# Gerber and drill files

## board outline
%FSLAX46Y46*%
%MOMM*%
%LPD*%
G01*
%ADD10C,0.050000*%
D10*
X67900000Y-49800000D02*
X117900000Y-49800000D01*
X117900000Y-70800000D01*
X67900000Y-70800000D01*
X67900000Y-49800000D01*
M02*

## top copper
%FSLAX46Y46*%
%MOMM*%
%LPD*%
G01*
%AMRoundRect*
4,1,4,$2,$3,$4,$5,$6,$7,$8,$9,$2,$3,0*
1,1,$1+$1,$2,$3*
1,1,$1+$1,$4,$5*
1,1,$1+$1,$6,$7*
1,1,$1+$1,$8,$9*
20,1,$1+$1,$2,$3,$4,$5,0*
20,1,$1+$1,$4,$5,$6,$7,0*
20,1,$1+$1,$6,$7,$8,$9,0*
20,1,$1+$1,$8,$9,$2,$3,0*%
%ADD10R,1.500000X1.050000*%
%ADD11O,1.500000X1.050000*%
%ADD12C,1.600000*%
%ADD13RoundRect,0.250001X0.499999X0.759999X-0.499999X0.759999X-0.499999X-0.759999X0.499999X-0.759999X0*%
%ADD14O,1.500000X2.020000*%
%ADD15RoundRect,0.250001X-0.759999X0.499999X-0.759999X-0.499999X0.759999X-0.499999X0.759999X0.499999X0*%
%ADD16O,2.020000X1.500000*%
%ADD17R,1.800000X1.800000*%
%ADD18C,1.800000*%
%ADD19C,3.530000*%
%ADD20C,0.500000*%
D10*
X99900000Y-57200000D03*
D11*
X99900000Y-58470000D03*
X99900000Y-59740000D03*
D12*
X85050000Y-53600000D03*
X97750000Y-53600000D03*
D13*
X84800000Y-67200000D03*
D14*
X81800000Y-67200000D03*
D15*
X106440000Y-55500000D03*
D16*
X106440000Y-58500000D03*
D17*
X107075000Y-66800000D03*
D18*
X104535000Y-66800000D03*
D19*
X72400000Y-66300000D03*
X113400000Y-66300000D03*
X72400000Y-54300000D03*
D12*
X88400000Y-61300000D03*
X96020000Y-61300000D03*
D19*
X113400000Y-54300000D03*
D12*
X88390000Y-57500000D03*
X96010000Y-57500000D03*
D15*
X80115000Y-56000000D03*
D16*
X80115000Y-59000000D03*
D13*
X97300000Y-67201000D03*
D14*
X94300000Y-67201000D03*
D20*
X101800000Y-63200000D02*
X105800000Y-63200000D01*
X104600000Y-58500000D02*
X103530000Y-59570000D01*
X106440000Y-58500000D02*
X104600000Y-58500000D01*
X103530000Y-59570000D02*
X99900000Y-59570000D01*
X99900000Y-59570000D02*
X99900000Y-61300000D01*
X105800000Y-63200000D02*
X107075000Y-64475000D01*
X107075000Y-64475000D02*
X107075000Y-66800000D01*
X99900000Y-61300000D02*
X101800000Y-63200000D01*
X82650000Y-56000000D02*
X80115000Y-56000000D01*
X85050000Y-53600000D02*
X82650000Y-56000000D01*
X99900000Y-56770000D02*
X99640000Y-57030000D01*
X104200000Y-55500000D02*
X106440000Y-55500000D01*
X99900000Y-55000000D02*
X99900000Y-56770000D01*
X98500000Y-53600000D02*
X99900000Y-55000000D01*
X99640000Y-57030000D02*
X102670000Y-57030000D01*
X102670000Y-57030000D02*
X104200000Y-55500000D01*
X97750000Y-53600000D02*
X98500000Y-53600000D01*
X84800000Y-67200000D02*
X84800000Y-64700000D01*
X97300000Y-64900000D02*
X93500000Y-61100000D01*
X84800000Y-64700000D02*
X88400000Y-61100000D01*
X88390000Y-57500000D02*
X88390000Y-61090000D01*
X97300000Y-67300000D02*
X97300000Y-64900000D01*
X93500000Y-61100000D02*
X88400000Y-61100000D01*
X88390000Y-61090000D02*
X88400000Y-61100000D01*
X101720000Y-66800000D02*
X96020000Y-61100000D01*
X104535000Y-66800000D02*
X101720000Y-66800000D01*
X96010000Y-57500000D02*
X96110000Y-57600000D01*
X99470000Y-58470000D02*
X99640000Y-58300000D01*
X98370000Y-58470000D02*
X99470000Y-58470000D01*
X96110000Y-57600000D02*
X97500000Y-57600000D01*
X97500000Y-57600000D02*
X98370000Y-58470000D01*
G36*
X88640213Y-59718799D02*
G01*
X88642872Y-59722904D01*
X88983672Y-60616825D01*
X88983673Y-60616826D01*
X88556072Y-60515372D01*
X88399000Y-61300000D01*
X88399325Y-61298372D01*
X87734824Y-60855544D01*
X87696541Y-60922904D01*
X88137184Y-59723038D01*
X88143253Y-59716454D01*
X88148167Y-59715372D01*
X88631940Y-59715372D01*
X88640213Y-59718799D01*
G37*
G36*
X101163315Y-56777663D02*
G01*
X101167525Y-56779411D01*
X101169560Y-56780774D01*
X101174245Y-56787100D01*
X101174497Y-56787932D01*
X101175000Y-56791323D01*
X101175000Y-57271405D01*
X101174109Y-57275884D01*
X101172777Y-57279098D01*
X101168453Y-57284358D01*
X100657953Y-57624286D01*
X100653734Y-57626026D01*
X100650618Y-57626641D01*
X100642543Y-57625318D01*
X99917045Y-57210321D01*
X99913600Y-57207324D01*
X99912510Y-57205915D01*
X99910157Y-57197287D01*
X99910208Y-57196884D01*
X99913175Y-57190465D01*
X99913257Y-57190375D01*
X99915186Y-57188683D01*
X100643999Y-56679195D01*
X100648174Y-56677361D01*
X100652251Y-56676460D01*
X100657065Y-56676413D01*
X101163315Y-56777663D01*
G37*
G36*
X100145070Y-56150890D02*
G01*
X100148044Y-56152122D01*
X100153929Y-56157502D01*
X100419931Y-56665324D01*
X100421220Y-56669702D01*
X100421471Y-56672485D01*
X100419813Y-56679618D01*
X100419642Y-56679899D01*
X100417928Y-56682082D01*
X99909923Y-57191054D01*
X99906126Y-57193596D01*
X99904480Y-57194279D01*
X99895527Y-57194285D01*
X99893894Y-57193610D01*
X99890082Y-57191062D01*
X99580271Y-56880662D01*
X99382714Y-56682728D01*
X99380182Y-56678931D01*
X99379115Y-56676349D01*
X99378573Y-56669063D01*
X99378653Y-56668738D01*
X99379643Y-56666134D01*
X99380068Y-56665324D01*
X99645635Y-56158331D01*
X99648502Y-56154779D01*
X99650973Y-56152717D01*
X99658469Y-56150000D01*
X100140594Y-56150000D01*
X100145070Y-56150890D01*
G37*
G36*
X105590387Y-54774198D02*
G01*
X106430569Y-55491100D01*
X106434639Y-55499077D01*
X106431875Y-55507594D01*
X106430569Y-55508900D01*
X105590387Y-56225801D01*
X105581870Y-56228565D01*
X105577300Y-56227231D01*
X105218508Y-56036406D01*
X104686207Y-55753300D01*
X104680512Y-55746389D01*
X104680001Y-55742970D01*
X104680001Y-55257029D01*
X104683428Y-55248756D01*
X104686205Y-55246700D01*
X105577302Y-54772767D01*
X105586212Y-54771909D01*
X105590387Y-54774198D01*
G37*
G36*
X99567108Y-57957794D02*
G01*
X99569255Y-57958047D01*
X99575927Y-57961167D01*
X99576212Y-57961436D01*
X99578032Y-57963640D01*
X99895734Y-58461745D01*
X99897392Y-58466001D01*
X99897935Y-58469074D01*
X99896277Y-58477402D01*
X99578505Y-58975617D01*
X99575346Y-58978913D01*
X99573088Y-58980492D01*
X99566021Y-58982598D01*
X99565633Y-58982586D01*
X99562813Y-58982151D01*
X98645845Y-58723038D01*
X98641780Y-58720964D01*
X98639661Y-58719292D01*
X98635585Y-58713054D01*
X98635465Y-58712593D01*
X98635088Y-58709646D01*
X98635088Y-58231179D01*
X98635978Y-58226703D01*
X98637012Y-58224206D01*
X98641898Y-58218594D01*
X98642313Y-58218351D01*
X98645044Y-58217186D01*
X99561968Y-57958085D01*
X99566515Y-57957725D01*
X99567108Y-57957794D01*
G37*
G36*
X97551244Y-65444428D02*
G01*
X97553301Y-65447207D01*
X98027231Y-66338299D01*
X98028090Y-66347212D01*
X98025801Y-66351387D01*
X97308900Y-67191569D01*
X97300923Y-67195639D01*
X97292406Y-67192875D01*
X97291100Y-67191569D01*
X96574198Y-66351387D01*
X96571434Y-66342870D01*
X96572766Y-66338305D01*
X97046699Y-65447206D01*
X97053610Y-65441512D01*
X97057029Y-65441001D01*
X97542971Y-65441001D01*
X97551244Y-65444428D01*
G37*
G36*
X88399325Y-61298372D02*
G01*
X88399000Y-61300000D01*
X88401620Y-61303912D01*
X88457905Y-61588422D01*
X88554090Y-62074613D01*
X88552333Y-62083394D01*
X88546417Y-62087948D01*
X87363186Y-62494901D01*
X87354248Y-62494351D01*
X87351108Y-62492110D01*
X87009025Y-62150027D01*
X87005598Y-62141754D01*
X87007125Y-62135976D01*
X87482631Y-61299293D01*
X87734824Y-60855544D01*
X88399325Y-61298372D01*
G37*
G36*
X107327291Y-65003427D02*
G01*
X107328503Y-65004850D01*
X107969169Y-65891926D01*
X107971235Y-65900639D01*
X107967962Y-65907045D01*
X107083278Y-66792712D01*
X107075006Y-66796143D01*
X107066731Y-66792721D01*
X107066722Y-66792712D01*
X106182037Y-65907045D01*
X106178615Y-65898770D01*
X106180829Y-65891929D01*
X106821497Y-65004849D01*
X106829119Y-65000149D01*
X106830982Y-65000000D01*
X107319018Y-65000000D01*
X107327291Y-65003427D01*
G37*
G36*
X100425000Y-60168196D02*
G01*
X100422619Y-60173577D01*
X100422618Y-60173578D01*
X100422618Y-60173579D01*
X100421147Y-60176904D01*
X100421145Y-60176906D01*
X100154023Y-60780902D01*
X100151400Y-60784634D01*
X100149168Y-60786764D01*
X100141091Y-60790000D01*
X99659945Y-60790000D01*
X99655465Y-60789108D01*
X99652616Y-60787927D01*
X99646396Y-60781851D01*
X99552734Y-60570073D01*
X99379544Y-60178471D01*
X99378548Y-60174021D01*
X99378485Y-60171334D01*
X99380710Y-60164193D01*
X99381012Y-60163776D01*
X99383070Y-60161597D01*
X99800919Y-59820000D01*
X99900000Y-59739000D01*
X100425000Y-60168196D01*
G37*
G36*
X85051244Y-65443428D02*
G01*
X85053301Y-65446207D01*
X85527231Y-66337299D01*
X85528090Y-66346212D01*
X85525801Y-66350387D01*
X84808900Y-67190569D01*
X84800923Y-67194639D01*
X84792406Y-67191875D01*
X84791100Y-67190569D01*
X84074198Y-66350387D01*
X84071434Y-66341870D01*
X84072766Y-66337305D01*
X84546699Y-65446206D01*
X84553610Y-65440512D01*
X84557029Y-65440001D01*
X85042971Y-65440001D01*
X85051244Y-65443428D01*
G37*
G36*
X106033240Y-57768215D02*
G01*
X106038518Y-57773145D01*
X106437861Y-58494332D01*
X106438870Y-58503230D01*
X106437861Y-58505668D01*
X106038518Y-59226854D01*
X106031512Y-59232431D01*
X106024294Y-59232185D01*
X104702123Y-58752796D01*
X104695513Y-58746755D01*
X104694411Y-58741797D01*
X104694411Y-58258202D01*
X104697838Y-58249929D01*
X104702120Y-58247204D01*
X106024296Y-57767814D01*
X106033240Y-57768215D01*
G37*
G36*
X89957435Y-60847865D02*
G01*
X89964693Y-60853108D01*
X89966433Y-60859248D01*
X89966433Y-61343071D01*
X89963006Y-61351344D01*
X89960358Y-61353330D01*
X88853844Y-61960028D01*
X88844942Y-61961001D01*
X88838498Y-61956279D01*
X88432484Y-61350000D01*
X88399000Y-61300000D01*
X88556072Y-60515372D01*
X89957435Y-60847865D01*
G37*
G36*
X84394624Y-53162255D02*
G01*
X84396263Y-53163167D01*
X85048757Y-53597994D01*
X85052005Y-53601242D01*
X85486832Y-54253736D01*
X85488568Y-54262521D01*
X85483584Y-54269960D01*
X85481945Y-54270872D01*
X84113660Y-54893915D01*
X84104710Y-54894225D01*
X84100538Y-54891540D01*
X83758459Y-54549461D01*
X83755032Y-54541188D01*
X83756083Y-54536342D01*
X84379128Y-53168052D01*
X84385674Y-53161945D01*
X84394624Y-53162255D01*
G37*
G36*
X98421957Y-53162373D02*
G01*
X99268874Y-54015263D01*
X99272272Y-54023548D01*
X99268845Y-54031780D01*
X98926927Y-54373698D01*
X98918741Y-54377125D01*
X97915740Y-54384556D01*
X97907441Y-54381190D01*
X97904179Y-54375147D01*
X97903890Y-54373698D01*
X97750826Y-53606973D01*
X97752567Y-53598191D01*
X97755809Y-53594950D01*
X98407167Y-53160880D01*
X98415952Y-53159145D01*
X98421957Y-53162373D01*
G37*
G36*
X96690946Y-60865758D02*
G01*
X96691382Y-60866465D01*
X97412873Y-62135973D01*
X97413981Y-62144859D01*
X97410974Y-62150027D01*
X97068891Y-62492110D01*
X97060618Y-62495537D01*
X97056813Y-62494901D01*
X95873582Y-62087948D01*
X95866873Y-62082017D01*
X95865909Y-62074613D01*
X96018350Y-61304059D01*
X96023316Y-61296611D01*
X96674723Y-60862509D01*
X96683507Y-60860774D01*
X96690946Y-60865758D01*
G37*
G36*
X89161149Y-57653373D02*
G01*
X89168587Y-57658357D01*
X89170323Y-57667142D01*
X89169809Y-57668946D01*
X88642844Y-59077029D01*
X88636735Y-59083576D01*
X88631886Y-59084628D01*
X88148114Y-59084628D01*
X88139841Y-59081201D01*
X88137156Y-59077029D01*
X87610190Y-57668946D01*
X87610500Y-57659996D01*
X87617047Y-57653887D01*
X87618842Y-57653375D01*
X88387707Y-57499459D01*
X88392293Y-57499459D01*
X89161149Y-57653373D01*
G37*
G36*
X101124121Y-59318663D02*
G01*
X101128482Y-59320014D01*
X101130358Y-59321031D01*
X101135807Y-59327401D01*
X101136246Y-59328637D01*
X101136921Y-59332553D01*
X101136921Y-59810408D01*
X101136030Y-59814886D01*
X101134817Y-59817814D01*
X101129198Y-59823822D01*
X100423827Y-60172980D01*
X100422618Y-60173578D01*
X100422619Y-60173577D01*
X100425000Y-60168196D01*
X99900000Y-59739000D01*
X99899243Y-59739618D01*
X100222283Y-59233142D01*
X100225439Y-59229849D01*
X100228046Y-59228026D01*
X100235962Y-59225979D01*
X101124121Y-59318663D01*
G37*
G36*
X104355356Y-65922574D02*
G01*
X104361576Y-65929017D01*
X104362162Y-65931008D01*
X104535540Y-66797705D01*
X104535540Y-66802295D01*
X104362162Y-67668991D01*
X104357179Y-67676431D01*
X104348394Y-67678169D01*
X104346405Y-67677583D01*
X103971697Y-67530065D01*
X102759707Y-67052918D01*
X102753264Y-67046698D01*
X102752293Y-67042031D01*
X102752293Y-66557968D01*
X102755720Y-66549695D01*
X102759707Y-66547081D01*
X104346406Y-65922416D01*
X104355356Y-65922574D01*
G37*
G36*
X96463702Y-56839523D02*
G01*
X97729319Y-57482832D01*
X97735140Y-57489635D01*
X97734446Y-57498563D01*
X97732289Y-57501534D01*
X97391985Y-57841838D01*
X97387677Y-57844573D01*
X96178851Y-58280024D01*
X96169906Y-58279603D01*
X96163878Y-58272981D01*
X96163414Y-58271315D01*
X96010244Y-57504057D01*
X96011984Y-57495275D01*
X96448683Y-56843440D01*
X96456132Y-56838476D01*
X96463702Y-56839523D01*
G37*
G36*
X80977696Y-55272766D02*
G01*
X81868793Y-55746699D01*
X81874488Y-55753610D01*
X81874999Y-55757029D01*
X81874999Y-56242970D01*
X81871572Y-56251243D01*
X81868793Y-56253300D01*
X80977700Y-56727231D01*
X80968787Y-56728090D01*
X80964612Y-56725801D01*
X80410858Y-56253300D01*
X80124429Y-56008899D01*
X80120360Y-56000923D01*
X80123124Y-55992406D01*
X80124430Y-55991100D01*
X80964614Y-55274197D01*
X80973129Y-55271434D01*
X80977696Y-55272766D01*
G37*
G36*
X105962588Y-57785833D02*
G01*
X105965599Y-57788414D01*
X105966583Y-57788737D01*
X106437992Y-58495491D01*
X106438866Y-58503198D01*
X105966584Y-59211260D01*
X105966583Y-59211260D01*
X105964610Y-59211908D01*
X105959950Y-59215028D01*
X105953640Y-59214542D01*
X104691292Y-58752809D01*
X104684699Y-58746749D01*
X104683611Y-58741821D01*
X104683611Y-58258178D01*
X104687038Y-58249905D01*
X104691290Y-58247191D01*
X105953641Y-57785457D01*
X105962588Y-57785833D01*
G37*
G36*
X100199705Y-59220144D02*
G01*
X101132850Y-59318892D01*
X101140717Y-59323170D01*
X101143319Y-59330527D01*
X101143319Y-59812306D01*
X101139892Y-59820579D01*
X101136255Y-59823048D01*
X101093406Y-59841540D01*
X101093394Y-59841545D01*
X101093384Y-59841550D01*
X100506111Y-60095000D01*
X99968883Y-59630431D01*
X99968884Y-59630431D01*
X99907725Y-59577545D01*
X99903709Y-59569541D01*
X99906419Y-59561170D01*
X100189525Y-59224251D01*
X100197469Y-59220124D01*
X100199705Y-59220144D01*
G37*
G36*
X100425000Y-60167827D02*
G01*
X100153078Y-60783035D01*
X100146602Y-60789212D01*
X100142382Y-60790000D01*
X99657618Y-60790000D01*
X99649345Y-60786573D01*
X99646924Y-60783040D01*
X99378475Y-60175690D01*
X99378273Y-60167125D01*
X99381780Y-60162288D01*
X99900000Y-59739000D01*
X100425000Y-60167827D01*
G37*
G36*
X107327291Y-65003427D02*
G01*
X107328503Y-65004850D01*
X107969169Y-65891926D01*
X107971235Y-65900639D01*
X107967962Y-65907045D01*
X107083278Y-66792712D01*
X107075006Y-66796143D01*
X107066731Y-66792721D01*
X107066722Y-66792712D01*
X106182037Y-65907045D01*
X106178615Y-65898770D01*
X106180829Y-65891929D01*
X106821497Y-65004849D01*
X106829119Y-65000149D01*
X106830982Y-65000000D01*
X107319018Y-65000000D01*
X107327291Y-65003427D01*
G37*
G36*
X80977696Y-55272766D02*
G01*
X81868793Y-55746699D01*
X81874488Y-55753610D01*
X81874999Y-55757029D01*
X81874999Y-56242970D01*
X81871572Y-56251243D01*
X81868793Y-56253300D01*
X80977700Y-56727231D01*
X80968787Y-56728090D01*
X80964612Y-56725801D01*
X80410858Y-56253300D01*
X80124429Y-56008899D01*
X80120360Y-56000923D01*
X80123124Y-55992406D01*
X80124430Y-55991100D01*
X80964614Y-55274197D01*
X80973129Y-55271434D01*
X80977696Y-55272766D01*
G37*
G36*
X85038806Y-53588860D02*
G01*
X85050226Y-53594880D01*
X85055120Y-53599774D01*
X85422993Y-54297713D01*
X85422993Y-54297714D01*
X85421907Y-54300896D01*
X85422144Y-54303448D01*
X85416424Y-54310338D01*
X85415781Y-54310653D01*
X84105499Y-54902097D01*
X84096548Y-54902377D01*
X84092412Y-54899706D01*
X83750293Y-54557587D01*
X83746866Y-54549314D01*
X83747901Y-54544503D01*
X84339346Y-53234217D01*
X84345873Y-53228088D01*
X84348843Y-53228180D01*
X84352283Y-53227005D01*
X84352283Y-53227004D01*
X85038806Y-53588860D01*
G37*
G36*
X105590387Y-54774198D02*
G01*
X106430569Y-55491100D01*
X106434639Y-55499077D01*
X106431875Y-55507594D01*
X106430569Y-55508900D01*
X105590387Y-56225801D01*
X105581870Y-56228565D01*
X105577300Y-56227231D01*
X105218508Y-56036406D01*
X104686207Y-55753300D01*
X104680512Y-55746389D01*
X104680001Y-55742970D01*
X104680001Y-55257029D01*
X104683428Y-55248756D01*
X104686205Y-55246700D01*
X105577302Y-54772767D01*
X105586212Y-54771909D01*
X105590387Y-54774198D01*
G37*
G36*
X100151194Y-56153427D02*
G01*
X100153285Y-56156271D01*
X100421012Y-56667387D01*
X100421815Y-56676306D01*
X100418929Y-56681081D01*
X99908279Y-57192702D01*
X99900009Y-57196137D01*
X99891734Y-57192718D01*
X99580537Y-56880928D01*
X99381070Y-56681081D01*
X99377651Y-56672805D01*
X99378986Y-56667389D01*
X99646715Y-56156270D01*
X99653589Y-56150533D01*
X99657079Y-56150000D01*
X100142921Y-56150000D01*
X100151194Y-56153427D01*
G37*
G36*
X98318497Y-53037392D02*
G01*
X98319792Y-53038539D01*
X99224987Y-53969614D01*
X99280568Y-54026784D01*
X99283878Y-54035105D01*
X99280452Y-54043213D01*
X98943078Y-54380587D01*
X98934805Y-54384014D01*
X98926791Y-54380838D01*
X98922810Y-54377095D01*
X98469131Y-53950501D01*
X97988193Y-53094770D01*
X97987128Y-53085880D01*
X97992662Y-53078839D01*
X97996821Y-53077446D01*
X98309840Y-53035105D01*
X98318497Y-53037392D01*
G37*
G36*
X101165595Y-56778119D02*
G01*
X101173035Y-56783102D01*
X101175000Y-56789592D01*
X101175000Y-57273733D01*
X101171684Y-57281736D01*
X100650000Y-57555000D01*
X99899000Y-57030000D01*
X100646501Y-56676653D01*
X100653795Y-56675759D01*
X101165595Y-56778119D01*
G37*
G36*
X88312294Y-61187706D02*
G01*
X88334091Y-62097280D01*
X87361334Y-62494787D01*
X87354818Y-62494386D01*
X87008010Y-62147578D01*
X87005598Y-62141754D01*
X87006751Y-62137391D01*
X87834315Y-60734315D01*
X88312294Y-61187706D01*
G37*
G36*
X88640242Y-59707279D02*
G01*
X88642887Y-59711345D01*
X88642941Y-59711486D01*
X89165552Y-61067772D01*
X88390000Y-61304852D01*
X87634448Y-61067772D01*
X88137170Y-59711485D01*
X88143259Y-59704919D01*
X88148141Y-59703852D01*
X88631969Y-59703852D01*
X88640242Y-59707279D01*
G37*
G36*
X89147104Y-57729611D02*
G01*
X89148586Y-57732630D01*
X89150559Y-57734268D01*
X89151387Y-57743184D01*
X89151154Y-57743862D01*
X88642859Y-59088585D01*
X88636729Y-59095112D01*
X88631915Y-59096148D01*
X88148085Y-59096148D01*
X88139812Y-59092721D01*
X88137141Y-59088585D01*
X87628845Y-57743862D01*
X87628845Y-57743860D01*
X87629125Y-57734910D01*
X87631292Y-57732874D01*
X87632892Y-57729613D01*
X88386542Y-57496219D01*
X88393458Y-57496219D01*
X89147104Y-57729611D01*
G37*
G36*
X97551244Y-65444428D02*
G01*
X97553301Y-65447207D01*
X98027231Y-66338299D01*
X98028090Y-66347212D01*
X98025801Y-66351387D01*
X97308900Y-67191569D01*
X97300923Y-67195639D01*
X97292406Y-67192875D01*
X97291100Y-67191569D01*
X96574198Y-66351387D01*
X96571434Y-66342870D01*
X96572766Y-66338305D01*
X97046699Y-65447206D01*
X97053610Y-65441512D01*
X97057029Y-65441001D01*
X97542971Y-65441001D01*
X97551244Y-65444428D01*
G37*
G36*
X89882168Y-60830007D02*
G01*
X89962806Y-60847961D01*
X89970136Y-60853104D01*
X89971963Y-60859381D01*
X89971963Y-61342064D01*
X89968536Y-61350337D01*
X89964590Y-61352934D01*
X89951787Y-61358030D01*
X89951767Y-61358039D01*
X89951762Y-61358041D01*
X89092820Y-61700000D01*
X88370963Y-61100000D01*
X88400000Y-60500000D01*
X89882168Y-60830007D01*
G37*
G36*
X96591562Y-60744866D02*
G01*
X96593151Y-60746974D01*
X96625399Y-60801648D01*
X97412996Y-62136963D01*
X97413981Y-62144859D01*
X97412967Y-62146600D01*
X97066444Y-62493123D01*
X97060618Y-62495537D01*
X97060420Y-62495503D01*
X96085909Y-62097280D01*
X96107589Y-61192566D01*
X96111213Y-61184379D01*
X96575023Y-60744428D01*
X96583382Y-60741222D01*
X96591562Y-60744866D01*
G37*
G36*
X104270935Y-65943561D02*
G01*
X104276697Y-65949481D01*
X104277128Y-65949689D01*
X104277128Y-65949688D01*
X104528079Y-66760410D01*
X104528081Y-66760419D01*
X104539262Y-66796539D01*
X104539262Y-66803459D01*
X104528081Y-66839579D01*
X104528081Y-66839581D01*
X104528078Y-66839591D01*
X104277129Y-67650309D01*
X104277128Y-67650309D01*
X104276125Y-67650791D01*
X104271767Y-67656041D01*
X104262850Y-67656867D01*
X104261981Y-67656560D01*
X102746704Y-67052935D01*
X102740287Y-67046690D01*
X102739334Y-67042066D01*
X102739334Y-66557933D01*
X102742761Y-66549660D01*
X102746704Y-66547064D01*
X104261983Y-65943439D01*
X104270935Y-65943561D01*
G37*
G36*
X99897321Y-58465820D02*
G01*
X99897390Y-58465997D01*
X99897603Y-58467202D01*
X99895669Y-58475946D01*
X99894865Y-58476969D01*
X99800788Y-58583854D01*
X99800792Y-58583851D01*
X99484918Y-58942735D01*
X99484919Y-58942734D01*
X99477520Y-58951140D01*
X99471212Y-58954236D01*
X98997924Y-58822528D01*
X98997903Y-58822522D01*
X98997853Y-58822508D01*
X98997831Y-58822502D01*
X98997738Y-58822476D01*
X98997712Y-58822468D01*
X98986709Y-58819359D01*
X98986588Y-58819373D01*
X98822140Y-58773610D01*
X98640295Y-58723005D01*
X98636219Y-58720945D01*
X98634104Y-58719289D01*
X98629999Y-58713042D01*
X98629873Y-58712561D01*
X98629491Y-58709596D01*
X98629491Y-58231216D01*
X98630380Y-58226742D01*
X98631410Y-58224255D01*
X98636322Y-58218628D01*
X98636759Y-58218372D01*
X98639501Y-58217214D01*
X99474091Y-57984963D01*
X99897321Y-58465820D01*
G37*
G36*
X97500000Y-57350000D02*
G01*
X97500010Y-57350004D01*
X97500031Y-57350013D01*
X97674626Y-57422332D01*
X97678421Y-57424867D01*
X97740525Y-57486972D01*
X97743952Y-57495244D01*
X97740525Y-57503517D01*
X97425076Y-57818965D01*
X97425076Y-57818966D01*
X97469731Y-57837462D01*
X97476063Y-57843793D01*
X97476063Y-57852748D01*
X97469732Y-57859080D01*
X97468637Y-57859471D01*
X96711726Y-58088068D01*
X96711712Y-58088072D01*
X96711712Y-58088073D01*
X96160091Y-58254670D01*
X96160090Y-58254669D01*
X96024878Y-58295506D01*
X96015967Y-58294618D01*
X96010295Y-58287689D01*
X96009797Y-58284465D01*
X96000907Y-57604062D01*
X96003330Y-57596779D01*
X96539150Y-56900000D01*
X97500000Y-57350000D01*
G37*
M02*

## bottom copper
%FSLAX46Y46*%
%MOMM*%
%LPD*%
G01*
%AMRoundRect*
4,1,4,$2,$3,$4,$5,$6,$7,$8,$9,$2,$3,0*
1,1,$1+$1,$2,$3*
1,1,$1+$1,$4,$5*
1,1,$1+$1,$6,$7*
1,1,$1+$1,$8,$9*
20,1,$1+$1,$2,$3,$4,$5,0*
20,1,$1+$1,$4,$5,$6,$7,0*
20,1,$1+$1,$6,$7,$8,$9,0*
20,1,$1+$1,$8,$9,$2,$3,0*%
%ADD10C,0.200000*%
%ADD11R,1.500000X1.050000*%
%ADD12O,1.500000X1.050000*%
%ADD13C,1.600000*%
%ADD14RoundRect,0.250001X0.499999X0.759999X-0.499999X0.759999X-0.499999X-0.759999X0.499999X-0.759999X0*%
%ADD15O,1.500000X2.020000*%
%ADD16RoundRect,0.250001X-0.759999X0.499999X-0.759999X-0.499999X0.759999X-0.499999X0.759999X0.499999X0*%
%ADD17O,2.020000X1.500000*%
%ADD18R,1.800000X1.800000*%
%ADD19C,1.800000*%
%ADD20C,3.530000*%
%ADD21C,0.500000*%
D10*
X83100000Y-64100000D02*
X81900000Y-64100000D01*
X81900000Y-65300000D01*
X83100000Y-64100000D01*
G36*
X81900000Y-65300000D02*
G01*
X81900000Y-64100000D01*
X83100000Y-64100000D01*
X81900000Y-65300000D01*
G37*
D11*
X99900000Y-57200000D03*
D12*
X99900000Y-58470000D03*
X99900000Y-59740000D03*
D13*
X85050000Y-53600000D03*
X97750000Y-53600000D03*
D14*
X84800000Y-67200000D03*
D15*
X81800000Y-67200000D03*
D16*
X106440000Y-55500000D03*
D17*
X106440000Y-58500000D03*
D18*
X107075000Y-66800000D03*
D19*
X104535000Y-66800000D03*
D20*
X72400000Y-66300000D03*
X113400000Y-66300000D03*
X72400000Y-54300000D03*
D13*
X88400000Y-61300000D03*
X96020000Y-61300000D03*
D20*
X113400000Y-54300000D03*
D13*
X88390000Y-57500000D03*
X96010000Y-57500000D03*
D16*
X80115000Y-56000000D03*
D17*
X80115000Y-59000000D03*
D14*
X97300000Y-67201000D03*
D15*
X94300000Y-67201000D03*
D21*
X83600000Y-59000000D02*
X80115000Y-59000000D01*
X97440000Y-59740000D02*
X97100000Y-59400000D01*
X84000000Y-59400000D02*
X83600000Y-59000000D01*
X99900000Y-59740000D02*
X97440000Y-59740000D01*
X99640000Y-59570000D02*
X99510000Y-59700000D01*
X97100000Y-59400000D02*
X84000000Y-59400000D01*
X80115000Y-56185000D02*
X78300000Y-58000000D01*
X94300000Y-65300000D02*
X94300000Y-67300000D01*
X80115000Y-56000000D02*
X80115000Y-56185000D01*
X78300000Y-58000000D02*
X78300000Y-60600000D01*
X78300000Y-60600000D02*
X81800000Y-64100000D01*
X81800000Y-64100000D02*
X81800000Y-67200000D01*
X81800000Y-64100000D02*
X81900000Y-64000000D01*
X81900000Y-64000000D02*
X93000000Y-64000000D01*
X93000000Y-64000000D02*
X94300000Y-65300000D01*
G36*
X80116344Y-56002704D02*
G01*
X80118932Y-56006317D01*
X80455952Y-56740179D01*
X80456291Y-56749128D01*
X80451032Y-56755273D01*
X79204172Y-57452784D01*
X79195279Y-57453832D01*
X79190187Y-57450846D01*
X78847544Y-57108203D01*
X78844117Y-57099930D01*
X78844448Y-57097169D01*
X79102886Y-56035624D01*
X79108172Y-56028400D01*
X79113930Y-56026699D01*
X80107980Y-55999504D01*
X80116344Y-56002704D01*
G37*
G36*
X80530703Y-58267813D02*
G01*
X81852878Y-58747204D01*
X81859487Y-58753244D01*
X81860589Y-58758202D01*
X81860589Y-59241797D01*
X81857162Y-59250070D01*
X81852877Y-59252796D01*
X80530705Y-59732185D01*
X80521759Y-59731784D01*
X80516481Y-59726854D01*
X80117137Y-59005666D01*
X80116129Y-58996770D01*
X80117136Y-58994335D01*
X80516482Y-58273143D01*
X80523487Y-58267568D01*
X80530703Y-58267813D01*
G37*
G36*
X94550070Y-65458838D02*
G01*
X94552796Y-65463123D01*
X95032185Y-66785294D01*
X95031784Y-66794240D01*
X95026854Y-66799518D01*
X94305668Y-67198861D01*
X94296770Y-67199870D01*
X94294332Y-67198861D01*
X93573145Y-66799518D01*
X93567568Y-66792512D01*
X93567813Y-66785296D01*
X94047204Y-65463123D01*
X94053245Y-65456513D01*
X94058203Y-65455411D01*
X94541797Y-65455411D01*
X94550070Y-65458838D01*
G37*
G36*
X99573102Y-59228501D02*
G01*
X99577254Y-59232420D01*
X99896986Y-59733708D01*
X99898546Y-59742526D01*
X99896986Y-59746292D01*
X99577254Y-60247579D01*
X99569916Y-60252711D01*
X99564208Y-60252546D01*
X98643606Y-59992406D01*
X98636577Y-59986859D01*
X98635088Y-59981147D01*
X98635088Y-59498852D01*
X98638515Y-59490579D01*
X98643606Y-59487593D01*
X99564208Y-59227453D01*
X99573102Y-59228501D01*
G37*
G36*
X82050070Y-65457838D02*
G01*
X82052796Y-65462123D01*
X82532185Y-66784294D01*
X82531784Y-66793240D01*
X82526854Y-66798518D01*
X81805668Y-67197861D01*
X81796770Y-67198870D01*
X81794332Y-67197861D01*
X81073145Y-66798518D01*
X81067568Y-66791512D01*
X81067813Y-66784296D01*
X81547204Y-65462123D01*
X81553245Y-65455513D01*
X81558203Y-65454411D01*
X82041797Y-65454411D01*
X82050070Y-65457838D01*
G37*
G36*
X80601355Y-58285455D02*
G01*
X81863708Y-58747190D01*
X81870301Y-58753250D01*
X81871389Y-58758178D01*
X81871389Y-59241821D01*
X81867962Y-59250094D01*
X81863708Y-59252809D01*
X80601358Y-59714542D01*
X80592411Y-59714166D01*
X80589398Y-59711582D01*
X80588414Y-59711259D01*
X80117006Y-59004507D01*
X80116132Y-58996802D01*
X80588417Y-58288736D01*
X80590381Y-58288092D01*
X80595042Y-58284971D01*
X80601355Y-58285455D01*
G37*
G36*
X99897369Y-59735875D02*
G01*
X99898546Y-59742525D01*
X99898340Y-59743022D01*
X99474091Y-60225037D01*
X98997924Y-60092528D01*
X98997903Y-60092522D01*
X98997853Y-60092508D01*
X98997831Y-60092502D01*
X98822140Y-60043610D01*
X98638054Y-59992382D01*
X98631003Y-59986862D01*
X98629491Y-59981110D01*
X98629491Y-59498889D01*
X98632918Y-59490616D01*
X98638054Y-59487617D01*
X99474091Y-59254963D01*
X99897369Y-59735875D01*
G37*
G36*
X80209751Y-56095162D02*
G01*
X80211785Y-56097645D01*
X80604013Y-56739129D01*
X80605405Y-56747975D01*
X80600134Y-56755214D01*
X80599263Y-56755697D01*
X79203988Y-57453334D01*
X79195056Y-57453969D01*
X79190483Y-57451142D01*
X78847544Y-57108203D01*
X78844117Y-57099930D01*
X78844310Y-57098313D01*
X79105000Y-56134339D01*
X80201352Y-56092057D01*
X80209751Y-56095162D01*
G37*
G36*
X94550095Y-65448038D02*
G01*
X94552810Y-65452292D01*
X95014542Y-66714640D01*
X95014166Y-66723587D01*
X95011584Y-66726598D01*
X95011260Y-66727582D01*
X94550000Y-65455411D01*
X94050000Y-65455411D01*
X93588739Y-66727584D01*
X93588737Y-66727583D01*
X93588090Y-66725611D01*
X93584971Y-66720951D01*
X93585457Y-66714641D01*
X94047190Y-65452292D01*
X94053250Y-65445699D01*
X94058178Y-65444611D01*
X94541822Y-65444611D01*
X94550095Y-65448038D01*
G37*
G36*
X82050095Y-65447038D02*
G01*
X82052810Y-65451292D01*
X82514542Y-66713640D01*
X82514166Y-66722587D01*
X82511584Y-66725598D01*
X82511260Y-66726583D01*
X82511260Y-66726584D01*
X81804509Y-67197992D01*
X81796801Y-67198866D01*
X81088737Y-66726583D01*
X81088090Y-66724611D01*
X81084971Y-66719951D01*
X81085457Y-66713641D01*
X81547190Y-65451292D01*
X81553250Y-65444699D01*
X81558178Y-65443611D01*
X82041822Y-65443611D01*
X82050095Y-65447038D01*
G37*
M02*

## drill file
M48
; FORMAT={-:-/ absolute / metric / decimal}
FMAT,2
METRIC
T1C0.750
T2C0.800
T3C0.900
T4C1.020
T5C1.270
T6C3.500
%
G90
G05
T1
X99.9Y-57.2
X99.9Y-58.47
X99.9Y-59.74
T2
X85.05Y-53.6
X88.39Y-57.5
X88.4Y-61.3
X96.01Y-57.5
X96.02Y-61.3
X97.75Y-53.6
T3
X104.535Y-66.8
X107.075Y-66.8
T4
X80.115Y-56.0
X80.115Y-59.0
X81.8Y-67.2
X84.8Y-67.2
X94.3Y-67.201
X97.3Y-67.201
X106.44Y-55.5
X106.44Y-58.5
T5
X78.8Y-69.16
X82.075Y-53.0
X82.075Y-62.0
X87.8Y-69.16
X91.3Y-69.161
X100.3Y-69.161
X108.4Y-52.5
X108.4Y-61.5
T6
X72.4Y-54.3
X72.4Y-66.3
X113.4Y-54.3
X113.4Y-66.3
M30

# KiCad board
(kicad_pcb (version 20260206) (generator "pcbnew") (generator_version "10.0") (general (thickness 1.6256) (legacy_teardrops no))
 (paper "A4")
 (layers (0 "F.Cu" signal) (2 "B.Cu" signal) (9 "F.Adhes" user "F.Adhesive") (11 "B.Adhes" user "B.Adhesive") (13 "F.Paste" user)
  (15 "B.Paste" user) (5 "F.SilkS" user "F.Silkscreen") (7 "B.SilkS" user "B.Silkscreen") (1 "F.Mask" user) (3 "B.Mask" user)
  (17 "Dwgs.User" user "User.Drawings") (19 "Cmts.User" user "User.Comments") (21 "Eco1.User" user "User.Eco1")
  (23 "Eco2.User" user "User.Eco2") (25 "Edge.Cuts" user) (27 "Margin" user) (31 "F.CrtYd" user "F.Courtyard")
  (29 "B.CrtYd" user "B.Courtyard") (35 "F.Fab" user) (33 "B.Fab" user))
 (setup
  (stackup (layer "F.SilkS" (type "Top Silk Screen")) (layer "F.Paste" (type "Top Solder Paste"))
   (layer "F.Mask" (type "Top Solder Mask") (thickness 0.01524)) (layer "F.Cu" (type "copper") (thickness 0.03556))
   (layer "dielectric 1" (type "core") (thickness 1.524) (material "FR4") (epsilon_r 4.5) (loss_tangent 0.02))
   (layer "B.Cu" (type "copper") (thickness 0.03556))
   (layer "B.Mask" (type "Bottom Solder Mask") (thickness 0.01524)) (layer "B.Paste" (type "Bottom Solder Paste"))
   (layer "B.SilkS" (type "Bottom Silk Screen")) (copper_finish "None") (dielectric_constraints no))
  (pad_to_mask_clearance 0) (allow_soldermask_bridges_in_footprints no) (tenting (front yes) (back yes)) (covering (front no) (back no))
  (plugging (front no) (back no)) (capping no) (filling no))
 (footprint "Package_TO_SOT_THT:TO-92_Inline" (layer "F.Cu") (at 99.9 57.2 -90)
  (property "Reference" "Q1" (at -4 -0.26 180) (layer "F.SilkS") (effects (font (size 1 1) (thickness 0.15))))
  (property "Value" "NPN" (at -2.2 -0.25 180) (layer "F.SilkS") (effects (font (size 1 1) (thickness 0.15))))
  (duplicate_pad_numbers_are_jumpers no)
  (pad "1" thru_hole rect (at 0 0 270) (size 1.05 1.5) (drill 0.75) (layers "*.Cu" "*.Mask") (remove_unused_layers no)
   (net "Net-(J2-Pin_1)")
   (teardrops (best_length_ratio 0.5) (max_length 1) (best_width_ratio 1) (max_width 2) (curved_edges no) (filter_ratio 0.9) (enabled yes)
    (allow_two_segments yes) (prefer_zone_connections yes)))
  (pad "2" thru_hole oval (at 1.27 0 270) (size 1.05 1.5) (drill 0.75) (layers "*.Cu" "*.Mask") (remove_unused_layers no) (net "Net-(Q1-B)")
   (teardrops (best_length_ratio 0.5) (max_length 1) (best_width_ratio 1) (max_width 2) (curved_edges no) (filter_ratio 0.9) (enabled yes)
    (allow_two_segments yes) (prefer_zone_connections yes)))
  (pad "3" thru_hole oval (at 2.54 0 270) (size 1.05 1.5) (drill 0.75) (layers "*.Cu" "*.Mask") (remove_unused_layers no) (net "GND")
   (teardrops (best_length_ratio 0.5) (max_length 1) (best_width_ratio 1) (max_width 2) (curved_edges no) (filter_ratio 0.9) (enabled yes)
    (allow_two_segments yes) (prefer_zone_connections yes))))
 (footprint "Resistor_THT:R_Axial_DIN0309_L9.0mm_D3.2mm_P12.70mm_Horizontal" (layer "F.Cu") (at 85.05 53.6)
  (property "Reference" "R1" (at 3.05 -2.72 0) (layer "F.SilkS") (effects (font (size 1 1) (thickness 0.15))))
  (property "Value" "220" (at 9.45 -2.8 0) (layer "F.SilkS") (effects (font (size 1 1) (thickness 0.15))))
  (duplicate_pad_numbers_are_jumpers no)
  (pad "1" thru_hole circle (at 0 0) (size 1.6 1.6) (drill 0.8) (layers "*.Cu" "*.Mask") (remove_unused_layers no) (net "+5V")
   (teardrops (best_length_ratio 0.5) (max_length 1) (best_width_ratio 1) (max_width 2) (curved_edges no) (filter_ratio 0.9) (enabled yes)
    (allow_two_segments yes) (prefer_zone_connections yes)))
  (pad "2" thru_hole circle (at 12.7 0) (size 1.6 1.6) (drill 0.8) (layers "*.Cu" "*.Mask") (remove_unused_layers no) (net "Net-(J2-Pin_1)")
   (teardrops (best_length_ratio 0.5) (max_length 1) (best_width_ratio 1) (max_width 2) (curved_edges no) (filter_ratio 0.9) (enabled yes)
    (allow_two_segments yes) (prefer_zone_connections yes))))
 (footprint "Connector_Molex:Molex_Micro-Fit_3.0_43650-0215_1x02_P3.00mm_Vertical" (layer "F.Cu") (at 84.8 67.2 180)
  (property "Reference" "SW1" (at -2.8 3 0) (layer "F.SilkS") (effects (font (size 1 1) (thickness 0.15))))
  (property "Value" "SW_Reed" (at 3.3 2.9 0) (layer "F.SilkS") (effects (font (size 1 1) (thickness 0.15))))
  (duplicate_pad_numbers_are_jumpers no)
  (pad "" np_thru_hole circle (at -3 -1.96 180) (size 1.27 1.27) (drill 1.27) (layers "*.Cu" "*.Mask"))
  (pad "" np_thru_hole circle (at 6 -1.96 180) (size 1.27 1.27) (drill 1.27) (layers "*.Cu" "*.Mask"))
  (pad "1" thru_hole roundrect (at 0 0 180) (size 1.5 2.02) (drill 1.02) (layers "*.Cu" "*.Mask") (remove_unused_layers no)
   (roundrect_rratio 0.166667) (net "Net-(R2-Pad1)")
   (teardrops (best_length_ratio 0.5) (max_length 1) (best_width_ratio 1) (max_width 2) (curved_edges no) (filter_ratio 0.9) (enabled yes)
    (allow_two_segments yes) (prefer_zone_connections yes)))
  (pad "2" thru_hole oval (at 3 0 180) (size 1.5 2.02) (drill 1.02) (layers "*.Cu" "*.Mask") (remove_unused_layers no) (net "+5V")
   (teardrops (best_length_ratio 0.5) (max_length 1) (best_width_ratio 1) (max_width 2) (curved_edges no) (filter_ratio 0.9) (enabled yes)
    (allow_two_segments yes) (prefer_zone_connections yes))))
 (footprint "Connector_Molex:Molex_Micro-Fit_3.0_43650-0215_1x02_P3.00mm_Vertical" (layer "F.Cu") (at 106.44 55.5 -90)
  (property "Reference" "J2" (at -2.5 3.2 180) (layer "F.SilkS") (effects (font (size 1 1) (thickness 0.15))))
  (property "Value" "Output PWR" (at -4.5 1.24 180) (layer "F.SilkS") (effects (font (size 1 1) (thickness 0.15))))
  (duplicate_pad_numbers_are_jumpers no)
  (pad "" np_thru_hole circle (at -3 -1.96 270) (size 1.27 1.27) (drill 1.27) (layers "*.Cu" "*.Mask"))
  (pad "" np_thru_hole circle (at 6 -1.96 270) (size 1.27 1.27) (drill 1.27) (layers "*.Cu" "*.Mask"))
  (pad "1" thru_hole roundrect (at 0 0 270) (size 1.5 2.02) (drill 1.02) (layers "*.Cu" "*.Mask") (remove_unused_layers no)
   (roundrect_rratio 0.166667) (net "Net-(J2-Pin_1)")
   (teardrops (best_length_ratio 0.5) (max_length 1) (best_width_ratio 1) (max_width 2) (curved_edges no) (filter_ratio 0.9) (enabled yes)
    (allow_two_segments yes) (prefer_zone_connections yes)))
  (pad "2" thru_hole oval (at 3 0 270) (size 1.5 2.02) (drill 1.02) (layers "*.Cu" "*.Mask") (remove_unused_layers no) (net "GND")
   (teardrops (best_length_ratio 0.5) (max_length 1) (best_width_ratio 1) (max_width 2) (curved_edges no) (filter_ratio 0.9) (enabled yes)
    (allow_two_segments yes) (prefer_zone_connections yes))))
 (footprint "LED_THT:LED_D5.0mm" (layer "F.Cu") (at 107.075 66.8 180)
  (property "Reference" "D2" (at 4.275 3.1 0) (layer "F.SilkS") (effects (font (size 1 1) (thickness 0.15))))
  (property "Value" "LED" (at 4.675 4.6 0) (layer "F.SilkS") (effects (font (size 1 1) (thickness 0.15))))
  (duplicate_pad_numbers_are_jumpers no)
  (pad "1" thru_hole rect (at 0 0 180) (size 1.8 1.8) (drill 0.9) (layers "*.Cu" "*.Mask") (remove_unused_layers no) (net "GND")
   (teardrops (best_length_ratio 0.5) (max_length 1) (best_width_ratio 1) (max_width 2) (curved_edges no) (filter_ratio 0.9) (enabled yes)
    (allow_two_segments yes) (prefer_zone_connections yes)))
  (pad "2" thru_hole circle (at 2.54 0 180) (size 1.8 1.8) (drill 0.9) (layers "*.Cu" "*.Mask") (remove_unused_layers no) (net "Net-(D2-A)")
   (teardrops (best_length_ratio 0.5) (max_length 1) (best_width_ratio 1) (max_width 2) (curved_edges no) (filter_ratio 0.9) (enabled yes)
    (allow_two_segments yes) (prefer_zone_connections yes))))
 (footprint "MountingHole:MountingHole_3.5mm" (layer "F.Cu") (at 72.4 66.3)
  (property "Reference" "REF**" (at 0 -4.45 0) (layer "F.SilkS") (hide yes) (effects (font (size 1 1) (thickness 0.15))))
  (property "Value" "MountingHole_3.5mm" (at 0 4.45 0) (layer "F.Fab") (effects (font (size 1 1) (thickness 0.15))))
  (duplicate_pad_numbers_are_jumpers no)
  (pad "" np_thru_hole circle (at 0 0) (size 3.53 3.53) (drill 3.5) (layers "*.Cu" "*.Mask")))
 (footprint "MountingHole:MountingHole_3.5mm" (layer "F.Cu") (at 113.4 66.3)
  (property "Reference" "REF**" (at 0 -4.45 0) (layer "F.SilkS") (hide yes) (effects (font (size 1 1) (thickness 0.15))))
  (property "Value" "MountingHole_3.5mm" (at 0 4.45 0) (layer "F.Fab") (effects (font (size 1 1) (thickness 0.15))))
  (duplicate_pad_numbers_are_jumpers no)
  (pad "" np_thru_hole circle (at 0 0) (size 3.53 3.53) (drill 3.5) (layers "*.Cu" "*.Mask")))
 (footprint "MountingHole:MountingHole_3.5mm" (layer "F.Cu") (at 72.4 54.3)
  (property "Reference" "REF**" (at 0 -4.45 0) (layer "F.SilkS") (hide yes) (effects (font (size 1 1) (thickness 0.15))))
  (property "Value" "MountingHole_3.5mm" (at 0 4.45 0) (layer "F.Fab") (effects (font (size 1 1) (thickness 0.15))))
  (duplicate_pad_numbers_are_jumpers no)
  (pad "" np_thru_hole circle (at 0 0) (size 3.53 3.53) (drill 3.5) (layers "*.Cu" "*.Mask")))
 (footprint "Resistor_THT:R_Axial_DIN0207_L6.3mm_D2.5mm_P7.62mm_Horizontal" (layer "F.Cu") (at 88.4 61.3)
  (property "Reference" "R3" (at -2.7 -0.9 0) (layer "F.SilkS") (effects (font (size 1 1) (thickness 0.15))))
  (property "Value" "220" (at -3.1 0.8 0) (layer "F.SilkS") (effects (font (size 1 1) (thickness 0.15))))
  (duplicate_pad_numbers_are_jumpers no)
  (pad "1" thru_hole circle (at 0 0) (size 1.6 1.6) (drill 0.8) (layers "*.Cu" "*.Mask") (remove_unused_layers no) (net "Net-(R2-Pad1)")
   (teardrops (best_length_ratio 0.5) (max_length 1) (best_width_ratio 1) (max_width 2) (curved_edges no) (filter_ratio 0.9) (enabled yes)
    (allow_two_segments yes) (prefer_zone_connections yes)))
  (pad "2" thru_hole circle (at 7.62 0) (size 1.6 1.6) (drill 0.8) (layers "*.Cu" "*.Mask") (remove_unused_layers no) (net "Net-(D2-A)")
   (teardrops (best_length_ratio 0.5) (max_length 1) (best_width_ratio 1) (max_width 2) (curved_edges no) (filter_ratio 0.9) (enabled yes)
    (allow_two_segments yes) (prefer_zone_connections yes))))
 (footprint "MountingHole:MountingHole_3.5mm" (layer "F.Cu") (at 113.4 54.3)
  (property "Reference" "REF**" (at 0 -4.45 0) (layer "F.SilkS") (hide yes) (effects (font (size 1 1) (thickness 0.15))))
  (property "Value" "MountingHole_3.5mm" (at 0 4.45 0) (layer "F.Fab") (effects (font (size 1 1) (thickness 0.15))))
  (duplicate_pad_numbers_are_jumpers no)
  (pad "" np_thru_hole circle (at 0 0) (size 3.53 3.53) (drill 3.5) (layers "*.Cu" "*.Mask")))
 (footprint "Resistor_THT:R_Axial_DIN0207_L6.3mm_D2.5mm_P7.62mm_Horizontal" (layer "F.Cu") (at 88.39 57.5)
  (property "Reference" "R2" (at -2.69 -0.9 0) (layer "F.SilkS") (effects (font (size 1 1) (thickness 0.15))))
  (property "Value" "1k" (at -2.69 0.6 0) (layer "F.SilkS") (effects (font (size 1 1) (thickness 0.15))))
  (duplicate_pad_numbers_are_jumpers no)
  (pad "1" thru_hole circle (at 0 0) (size 1.6 1.6) (drill 0.8) (layers "*.Cu" "*.Mask") (remove_unused_layers no) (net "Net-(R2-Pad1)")
   (teardrops (best_length_ratio 0.5) (max_length 1) (best_width_ratio 1) (max_width 2) (curved_edges no) (filter_ratio 0.9) (enabled yes)
    (allow_two_segments yes) (prefer_zone_connections yes)))
  (pad "2" thru_hole circle (at 7.62 0) (size 1.6 1.6) (drill 0.8) (layers "*.Cu" "*.Mask") (remove_unused_layers no) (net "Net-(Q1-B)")
   (teardrops (best_length_ratio 0.5) (max_length 1) (best_width_ratio 1) (max_width 2) (curved_edges no) (filter_ratio 0.9) (enabled yes)
    (allow_two_segments yes) (prefer_zone_connections yes))))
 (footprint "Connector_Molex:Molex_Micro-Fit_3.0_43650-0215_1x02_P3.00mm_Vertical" (layer "F.Cu") (at 80.115 56 -90)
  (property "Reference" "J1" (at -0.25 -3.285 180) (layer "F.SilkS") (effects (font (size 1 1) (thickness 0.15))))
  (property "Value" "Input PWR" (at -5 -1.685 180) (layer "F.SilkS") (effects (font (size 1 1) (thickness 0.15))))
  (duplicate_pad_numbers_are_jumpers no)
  (pad "" np_thru_hole circle (at -3 -1.96 270) (size 1.27 1.27) (drill 1.27) (layers "*.Cu" "*.Mask"))
  (pad "" np_thru_hole circle (at 6 -1.96 270) (size 1.27 1.27) (drill 1.27) (layers "*.Cu" "*.Mask"))
  (pad "1" thru_hole roundrect (at 0 0 270) (size 1.5 2.02) (drill 1.02) (layers "*.Cu" "*.Mask") (remove_unused_layers no)
   (roundrect_rratio 0.166667) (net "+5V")
   (teardrops (best_length_ratio 0.5) (max_length 1) (best_width_ratio 1) (max_width 2) (curved_edges no) (filter_ratio 0.9) (enabled yes)
    (allow_two_segments yes) (prefer_zone_connections yes)))
  (pad "2" thru_hole oval (at 3 0 270) (size 1.5 2.02) (drill 1.02) (layers "*.Cu" "*.Mask") (remove_unused_layers no) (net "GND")
   (teardrops (best_length_ratio 0.5) (max_length 1) (best_width_ratio 1) (max_width 2) (curved_edges no) (filter_ratio 0.9) (enabled yes)
    (allow_two_segments yes) (prefer_zone_connections yes))))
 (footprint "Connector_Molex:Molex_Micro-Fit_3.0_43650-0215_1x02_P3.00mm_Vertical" (layer "F.Cu") (at 97.3 67.201 180)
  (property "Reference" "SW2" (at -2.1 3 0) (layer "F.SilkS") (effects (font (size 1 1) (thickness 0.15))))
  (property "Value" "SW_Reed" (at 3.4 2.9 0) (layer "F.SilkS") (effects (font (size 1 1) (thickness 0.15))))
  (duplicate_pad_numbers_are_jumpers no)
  (pad "" np_thru_hole circle (at -3 -1.96 180) (size 1.27 1.27) (drill 1.27) (layers "*.Cu" "*.Mask"))
  (pad "" np_thru_hole circle (at 6 -1.96 180) (size 1.27 1.27) (drill 1.27) (layers "*.Cu" "*.Mask"))
  (pad "1" thru_hole roundrect (at 0 0 180) (size 1.5 2.02) (drill 1.02) (layers "*.Cu" "*.Mask") (remove_unused_layers no)
   (roundrect_rratio 0.166667) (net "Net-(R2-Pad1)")
   (teardrops (best_length_ratio 0.5) (max_length 1) (best_width_ratio 1) (max_width 2) (curved_edges no) (filter_ratio 0.9) (enabled yes)
    (allow_two_segments yes) (prefer_zone_connections yes)))
  (pad "2" thru_hole oval (at 3 0 180) (size 1.5 2.02) (drill 1.02) (layers "*.Cu" "*.Mask") (remove_unused_layers no) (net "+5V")
   (teardrops (best_length_ratio 0.5) (max_length 1) (best_width_ratio 1) (max_width 2) (curved_edges no) (filter_ratio 0.9) (enabled yes)
    (allow_two_segments yes) (prefer_zone_connections yes))))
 (gr_poly (pts (xy 83.1 64.1) (xy 81.9 64.1) (xy 81.9 65.3)) (stroke (width 0.2) (type solid)) (fill yes) (layer "B.Cu") (net "+5V"))
 (gr_rect (start 67.9 49.8) (end 117.9 70.8) (stroke (width 0.05) (type solid)) (fill no) (layer "Edge.Cuts"))
 (segment (start 101.8 63.2) (end 105.8 63.2) (width 0.5) (layer "F.Cu") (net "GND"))
 (segment (start 104.6 58.5) (end 103.53 59.57) (width 0.5) (layer "F.Cu") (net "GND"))
 (segment (start 106.44 58.5) (end 104.6 58.5) (width 0.5) (layer "F.Cu") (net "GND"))
 (segment (start 103.53 59.57) (end 99.9 59.57) (width 0.5) (layer "F.Cu") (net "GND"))
 (segment (start 99.9 59.57) (end 99.9 61.3) (width 0.5) (layer "F.Cu") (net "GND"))
 (segment (start 105.8 63.2) (end 107.075 64.475) (width 0.5) (layer "F.Cu") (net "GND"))
 (segment (start 107.075 64.475) (end 107.075 66.8) (width 0.5) (layer "F.Cu") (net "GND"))
 (segment (start 99.9 61.3) (end 101.8 63.2) (width 0.5) (layer "F.Cu") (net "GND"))
 (segment (start 83.6 59) (end 80.115 59) (width 0.5) (layer "B.Cu") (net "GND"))
 (segment (start 97.44 59.74) (end 97.1 59.4) (width 0.5) (layer "B.Cu") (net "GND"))
 (segment (start 84 59.4) (end 83.6 59) (width 0.5) (layer "B.Cu") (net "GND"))
 (segment (start 99.9 59.74) (end 97.44 59.74) (width 0.5) (layer "B.Cu") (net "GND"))
 (segment (start 99.64 59.57) (end 99.51 59.7) (width 0.5) (layer "B.Cu") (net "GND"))
 (segment (start 97.1 59.4) (end 84 59.4) (width 0.5) (layer "B.Cu") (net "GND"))
 (segment (start 82.65 56) (end 80.115 56) (width 0.5) (layer "F.Cu") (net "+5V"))
 (segment (start 85.05 53.6) (end 82.65 56) (width 0.5) (layer "F.Cu") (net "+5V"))
 (segment (start 80.115 56.185) (end 78.3 58) (width 0.5) (layer "B.Cu") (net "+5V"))
 (segment (start 94.3 65.3) (end 94.3 67.3) (width 0.5) (layer "B.Cu") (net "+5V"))
 (segment (start 80.115 56) (end 80.115 56.185) (width 0.5) (layer "B.Cu") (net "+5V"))
 (segment (start 78.3 58) (end 78.3 60.6) (width 0.5) (layer "B.Cu") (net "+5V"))
 (segment (start 78.3 60.6) (end 81.8 64.1) (width 0.5) (layer "B.Cu") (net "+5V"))
 (segment (start 81.8 64.1) (end 81.8 67.2) (width 0.5) (layer "B.Cu") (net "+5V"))
 (segment (start 81.8 64.1) (end 81.9 64) (width 0.5) (layer "B.Cu") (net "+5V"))
 (segment (start 81.9 64) (end 93 64) (width 0.5) (layer "B.Cu") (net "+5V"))
 (segment (start 93 64) (end 94.3 65.3) (width 0.5) (layer "B.Cu") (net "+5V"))
 (segment (start 99.9 56.77) (end 99.64 57.03) (width 0.5) (layer "F.Cu") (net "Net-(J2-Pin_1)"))
 (segment (start 104.2 55.5) (end 106.44 55.5) (width 0.5) (layer "F.Cu") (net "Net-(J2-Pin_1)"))
 (segment (start 99.9 55) (end 99.9 56.77) (width 0.5) (layer "F.Cu") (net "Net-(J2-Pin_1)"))
 (segment (start 98.5 53.6) (end 99.9 55) (width 0.5) (layer "F.Cu") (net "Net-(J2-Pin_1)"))
 (segment (start 99.64 57.03) (end 102.67 57.03) (width 0.5) (layer "F.Cu") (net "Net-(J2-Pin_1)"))
 (segment (start 102.67 57.03) (end 104.2 55.5) (width 0.5) (layer "F.Cu") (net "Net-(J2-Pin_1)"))
 (segment (start 97.75 53.6) (end 98.5 53.6) (width 0.5) (layer "F.Cu") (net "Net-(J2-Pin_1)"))
 (segment (start 84.8 67.2) (end 84.8 64.7) (width 0.5) (layer "F.Cu") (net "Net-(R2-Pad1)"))
 (segment (start 97.3 64.9) (end 93.5 61.1) (width 0.5) (layer "F.Cu") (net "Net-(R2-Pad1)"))
 (segment (start 84.8 64.7) (end 88.4 61.1) (width 0.5) (layer "F.Cu") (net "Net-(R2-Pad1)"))
 (segment (start 88.39 57.5) (end 88.39 61.09) (width 0.5) (layer "F.Cu") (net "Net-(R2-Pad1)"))
 (segment (start 97.3 67.3) (end 97.3 64.9) (width 0.5) (layer "F.Cu") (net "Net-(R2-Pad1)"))
 (segment (start 93.5 61.1) (end 88.4 61.1) (width 0.5) (layer "F.Cu") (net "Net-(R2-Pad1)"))
 (segment (start 88.39 61.09) (end 88.4 61.1) (width 0.5) (layer "F.Cu") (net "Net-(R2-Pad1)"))
 (segment (start 101.72 66.8) (end 96.02 61.1) (width 0.5) (layer "F.Cu") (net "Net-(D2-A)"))
 (segment (start 104.535 66.8) (end 101.72 66.8) (width 0.5) (layer "F.Cu") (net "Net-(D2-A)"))
 (segment (start 96.01 57.5) (end 96.11 57.6) (width 0.5) (layer "F.Cu") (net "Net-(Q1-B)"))
 (segment (start 99.47 58.47) (end 99.64 58.3) (width 0.5) (layer "F.Cu") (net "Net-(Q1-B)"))
 (segment (start 98.37 58.47) (end 99.47 58.47) (width 0.5) (layer "F.Cu") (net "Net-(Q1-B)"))
 (segment (start 96.11 57.6) (end 97.5 57.6) (width 0.5) (layer "F.Cu") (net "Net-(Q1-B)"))
 (segment (start 97.5 57.6) (end 98.37 58.47) (width 0.5) (layer "F.Cu") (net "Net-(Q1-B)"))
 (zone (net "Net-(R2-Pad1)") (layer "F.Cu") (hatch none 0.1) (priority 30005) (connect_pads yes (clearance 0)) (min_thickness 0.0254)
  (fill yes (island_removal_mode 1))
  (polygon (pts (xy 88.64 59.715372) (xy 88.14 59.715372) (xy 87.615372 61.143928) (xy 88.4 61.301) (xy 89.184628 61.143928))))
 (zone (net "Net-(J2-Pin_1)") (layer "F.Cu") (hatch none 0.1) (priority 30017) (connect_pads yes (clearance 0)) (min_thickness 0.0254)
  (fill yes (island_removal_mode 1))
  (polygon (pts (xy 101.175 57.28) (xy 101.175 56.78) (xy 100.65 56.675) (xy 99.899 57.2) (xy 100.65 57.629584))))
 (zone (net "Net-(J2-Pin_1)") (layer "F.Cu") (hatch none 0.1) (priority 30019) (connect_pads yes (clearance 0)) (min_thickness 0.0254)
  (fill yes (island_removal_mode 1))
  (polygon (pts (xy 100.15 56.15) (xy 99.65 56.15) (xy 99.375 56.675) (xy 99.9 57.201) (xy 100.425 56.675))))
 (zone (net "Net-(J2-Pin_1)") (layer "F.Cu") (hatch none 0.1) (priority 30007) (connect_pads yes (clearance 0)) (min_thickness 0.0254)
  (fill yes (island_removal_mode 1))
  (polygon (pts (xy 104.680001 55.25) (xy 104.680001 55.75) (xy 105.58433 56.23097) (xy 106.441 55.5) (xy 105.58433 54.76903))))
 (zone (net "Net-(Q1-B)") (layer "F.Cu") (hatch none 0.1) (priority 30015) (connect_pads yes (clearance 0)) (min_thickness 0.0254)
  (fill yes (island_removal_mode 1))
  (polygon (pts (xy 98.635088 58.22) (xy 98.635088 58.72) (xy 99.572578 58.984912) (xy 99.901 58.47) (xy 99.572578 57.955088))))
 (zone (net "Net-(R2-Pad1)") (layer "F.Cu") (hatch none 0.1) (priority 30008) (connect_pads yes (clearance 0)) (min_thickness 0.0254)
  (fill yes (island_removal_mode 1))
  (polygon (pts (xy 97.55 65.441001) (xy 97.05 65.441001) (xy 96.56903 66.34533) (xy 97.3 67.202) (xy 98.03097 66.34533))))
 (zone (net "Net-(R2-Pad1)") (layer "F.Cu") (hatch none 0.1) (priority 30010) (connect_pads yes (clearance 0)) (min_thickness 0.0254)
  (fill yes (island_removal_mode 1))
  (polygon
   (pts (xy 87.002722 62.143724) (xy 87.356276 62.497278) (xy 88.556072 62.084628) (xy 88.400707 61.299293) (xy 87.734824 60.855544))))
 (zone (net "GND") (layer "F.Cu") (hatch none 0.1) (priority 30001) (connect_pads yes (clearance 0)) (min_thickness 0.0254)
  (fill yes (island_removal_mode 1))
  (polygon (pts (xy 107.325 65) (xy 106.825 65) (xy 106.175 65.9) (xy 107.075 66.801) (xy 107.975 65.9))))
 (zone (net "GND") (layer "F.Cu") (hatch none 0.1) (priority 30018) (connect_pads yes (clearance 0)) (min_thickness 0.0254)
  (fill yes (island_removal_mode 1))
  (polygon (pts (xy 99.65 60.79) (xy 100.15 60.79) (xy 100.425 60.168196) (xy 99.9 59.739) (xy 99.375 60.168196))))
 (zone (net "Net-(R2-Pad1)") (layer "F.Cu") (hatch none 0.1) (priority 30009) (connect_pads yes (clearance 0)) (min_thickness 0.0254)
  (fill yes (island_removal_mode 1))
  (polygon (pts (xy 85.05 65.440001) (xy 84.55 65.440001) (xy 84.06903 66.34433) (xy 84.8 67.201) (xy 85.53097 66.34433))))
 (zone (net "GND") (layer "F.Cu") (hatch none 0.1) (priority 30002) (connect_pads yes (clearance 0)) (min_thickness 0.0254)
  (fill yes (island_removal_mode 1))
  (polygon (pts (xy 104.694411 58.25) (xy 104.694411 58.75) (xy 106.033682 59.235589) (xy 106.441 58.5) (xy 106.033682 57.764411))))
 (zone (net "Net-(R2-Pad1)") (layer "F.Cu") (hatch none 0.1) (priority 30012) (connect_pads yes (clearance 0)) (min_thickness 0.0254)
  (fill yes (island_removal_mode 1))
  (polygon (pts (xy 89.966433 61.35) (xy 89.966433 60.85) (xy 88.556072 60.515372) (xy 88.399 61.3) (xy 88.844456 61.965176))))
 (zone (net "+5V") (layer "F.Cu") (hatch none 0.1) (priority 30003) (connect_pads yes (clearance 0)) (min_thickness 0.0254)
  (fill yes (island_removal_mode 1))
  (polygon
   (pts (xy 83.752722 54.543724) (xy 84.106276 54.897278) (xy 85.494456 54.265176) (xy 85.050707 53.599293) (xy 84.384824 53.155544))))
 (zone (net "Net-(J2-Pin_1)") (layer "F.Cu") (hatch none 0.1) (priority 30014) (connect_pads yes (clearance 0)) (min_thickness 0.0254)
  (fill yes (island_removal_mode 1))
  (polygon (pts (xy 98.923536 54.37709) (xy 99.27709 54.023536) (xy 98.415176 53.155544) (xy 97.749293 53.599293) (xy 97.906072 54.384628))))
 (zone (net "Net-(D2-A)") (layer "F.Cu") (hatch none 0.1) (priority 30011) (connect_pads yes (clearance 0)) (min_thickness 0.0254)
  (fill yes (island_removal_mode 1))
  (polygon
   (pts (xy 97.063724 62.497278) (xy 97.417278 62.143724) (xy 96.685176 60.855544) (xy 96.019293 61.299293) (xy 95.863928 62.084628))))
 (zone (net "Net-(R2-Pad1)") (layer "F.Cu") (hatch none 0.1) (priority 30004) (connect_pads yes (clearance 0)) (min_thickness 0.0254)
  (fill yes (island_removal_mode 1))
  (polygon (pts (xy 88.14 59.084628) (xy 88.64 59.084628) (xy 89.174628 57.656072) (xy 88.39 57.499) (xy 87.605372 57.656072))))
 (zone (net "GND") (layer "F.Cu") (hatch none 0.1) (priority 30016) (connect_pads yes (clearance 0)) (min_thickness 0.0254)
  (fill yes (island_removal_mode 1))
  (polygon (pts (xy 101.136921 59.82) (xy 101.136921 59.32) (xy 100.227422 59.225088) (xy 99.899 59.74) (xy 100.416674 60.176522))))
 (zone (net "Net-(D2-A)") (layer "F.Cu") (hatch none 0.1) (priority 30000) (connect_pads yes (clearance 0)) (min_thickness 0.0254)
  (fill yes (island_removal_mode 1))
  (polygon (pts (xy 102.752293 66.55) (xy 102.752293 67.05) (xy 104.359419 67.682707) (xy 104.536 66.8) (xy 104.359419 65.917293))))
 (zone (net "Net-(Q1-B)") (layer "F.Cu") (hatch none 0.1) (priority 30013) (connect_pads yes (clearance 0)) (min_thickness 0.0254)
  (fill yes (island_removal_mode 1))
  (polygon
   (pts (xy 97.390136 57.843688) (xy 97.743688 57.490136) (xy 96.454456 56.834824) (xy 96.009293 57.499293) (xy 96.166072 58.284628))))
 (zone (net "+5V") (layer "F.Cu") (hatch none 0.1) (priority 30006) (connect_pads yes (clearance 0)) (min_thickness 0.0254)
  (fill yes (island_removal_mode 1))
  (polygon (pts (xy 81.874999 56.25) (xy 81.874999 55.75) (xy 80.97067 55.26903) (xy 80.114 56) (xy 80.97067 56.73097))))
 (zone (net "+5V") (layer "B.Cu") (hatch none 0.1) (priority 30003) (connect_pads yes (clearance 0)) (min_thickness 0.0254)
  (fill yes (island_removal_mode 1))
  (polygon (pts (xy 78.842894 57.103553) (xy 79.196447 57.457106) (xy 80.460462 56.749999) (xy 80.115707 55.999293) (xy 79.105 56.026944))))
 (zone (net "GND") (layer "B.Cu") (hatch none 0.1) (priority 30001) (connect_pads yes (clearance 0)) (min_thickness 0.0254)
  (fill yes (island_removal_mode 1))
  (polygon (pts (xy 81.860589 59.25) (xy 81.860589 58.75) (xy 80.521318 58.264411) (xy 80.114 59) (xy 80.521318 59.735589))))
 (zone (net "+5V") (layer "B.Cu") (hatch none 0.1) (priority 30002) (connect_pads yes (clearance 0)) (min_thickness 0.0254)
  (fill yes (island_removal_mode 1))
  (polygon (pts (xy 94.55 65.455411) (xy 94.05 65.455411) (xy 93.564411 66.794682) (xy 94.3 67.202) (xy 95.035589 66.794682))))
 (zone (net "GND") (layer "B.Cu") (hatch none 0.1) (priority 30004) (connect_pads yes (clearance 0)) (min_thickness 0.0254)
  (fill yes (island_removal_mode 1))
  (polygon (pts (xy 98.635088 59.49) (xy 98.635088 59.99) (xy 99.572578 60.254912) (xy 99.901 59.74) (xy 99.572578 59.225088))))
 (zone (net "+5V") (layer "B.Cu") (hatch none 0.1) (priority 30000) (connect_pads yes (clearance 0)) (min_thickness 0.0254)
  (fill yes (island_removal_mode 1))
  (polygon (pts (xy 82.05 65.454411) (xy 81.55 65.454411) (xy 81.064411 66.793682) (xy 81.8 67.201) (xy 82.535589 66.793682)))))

